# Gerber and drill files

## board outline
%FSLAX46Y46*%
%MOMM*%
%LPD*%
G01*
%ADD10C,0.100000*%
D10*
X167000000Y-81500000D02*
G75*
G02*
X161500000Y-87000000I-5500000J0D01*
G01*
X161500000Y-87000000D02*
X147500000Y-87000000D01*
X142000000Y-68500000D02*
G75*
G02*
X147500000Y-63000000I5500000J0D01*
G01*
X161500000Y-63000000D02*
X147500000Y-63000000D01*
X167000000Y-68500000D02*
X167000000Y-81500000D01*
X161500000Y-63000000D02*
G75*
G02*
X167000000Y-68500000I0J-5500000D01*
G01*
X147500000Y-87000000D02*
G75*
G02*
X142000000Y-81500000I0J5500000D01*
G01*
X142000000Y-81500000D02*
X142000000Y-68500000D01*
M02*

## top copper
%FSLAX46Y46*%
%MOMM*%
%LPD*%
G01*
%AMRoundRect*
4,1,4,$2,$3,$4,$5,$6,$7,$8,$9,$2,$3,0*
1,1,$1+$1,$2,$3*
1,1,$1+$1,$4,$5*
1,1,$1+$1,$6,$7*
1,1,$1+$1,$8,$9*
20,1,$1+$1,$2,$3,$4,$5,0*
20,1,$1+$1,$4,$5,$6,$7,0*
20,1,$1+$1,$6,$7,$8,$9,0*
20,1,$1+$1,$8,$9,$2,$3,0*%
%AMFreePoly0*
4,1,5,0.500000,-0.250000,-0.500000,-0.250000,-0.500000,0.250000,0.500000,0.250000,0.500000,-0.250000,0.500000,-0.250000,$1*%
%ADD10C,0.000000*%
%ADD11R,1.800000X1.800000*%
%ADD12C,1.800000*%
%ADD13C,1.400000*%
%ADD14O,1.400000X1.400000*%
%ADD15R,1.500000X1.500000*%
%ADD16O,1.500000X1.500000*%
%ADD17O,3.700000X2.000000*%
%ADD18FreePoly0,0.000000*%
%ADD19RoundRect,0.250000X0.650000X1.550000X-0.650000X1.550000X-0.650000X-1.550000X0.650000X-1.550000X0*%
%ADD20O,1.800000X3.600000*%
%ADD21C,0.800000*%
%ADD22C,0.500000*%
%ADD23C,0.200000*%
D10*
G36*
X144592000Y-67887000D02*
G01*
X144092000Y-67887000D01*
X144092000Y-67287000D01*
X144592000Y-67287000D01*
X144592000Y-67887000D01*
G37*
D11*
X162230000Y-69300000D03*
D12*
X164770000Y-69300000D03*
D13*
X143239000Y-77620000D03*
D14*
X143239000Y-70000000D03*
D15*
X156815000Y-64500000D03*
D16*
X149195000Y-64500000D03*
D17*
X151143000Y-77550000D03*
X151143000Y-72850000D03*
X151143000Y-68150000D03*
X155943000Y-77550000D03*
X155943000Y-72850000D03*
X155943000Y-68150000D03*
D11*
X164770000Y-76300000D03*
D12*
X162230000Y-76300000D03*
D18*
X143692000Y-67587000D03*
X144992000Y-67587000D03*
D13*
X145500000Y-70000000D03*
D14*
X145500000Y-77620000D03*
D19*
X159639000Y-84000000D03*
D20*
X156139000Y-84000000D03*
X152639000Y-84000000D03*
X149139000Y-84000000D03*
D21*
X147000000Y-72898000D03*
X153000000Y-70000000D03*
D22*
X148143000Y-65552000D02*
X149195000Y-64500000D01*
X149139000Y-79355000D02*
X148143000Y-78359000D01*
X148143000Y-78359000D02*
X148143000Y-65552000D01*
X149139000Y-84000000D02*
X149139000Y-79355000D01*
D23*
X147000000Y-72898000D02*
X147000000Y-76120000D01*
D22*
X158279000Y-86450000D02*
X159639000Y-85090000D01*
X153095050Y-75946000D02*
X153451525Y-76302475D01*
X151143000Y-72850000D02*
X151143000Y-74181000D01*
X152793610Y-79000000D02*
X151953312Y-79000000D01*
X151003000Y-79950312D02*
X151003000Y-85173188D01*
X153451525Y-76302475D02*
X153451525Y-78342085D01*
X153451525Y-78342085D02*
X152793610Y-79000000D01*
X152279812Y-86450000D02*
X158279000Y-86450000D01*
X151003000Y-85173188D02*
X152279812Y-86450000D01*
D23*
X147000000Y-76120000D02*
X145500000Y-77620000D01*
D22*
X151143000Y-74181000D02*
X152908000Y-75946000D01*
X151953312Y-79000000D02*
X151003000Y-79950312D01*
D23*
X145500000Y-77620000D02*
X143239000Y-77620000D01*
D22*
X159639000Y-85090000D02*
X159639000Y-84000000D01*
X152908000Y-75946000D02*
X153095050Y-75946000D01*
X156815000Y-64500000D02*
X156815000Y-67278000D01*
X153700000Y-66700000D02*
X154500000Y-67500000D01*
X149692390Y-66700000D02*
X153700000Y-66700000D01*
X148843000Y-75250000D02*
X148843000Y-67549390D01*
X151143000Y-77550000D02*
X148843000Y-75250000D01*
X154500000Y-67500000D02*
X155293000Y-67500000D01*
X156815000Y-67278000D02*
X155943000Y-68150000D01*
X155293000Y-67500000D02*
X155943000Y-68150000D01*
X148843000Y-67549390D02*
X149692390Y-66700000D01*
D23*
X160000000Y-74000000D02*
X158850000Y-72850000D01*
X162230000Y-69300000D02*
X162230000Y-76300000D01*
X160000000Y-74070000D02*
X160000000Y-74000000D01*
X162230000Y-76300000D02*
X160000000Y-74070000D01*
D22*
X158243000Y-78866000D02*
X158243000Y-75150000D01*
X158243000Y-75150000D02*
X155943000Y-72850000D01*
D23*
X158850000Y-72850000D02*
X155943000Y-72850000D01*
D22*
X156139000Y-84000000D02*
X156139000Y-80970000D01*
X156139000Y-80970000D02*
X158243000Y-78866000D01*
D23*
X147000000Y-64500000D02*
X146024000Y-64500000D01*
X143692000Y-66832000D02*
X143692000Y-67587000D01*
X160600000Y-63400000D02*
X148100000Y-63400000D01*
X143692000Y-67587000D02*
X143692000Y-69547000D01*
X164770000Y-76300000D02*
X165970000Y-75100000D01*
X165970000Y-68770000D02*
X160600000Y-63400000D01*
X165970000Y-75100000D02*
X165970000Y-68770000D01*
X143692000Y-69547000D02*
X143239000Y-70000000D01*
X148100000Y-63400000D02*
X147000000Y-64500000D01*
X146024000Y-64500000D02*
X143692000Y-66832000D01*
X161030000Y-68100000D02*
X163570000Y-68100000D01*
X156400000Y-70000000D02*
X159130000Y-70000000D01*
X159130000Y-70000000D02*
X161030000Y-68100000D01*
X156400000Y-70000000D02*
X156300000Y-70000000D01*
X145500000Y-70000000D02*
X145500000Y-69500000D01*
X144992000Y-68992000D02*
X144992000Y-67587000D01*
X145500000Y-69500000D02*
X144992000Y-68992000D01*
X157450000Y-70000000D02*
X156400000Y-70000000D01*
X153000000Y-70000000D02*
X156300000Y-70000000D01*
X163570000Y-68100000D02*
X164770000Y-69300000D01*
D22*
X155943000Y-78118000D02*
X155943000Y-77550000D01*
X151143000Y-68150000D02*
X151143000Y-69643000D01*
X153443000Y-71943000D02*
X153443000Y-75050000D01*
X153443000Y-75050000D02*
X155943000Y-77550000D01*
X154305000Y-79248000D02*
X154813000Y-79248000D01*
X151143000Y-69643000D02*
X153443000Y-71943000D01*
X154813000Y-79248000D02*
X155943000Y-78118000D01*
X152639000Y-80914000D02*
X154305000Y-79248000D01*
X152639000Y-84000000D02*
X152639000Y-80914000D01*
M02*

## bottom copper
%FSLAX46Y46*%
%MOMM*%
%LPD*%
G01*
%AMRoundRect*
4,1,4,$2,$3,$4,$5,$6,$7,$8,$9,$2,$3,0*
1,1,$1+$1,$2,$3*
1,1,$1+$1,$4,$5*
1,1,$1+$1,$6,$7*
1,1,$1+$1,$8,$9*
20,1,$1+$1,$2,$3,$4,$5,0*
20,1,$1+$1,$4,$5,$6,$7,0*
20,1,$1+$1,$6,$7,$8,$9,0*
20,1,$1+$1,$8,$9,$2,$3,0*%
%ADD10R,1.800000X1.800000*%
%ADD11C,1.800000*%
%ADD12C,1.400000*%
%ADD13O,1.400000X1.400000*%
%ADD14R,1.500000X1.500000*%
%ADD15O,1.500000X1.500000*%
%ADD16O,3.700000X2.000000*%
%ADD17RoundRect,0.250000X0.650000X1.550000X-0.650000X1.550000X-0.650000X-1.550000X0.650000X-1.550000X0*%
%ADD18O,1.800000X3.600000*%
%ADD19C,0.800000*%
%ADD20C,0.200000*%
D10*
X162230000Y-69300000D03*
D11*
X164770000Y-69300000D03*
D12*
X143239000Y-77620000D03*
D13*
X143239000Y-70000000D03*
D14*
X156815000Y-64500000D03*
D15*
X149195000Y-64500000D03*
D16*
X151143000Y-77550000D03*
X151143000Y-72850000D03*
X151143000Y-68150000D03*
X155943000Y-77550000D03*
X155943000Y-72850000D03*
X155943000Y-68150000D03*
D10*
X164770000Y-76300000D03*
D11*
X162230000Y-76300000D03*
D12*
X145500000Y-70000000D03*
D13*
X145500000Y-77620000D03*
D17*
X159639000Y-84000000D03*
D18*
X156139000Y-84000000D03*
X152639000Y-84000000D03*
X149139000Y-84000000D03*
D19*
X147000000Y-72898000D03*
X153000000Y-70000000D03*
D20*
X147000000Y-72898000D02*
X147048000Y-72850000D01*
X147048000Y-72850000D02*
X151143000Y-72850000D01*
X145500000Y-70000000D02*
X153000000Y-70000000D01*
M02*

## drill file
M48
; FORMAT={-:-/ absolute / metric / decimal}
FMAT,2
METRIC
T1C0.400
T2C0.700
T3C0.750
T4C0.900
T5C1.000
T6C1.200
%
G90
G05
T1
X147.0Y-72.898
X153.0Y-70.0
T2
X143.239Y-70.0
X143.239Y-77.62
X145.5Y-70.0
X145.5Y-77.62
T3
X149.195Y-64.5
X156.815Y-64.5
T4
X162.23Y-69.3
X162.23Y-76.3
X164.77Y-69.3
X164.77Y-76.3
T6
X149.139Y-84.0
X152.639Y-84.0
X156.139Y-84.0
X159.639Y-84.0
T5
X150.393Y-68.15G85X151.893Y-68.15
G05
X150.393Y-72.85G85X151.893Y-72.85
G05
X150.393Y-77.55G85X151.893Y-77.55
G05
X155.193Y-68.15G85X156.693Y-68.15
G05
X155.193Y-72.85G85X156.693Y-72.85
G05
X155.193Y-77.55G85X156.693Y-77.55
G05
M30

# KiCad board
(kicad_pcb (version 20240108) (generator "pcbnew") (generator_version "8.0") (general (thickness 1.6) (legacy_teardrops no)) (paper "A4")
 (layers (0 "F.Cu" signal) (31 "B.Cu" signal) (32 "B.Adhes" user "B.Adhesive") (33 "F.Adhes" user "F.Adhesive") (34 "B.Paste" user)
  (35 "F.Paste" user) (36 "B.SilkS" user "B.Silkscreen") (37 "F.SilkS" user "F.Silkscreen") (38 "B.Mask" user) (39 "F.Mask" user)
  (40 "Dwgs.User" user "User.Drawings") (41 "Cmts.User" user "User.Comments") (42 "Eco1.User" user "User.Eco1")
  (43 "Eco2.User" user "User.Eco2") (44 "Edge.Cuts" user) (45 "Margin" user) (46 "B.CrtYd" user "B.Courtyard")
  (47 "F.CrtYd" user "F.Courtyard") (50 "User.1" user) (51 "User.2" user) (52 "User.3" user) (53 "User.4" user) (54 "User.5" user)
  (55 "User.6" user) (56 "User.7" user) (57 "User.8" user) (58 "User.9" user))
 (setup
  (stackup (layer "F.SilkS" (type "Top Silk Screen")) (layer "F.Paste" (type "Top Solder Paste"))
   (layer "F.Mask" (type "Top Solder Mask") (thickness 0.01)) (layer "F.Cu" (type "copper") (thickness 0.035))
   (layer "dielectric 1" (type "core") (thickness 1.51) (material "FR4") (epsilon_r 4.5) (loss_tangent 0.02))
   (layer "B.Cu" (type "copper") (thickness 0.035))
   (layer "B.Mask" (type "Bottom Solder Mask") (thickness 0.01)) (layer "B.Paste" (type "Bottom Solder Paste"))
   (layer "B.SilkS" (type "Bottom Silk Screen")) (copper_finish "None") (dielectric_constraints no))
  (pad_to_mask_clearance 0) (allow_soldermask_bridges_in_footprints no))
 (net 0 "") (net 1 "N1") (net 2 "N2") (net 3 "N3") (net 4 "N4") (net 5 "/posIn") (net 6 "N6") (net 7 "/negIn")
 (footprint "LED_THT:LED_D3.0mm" (layer "F.Cu") (at 162.23 69.3)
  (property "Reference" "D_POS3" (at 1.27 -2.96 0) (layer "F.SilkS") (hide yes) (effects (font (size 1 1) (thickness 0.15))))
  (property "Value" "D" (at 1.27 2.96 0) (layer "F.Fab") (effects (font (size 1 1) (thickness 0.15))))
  (pad "1" thru_hole rect (at 0 0) (size 1.8 1.8) (drill 0.9) (layers "*.Cu" "*.Mask") (remove_unused_layers no) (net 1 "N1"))
  (pad "2" thru_hole circle (at 2.54 0) (size 1.8 1.8) (drill 0.9) (layers "*.Cu" "*.Mask") (remove_unused_layers no) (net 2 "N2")))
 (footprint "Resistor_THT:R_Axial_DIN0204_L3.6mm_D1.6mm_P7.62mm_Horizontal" (layer "F.Cu") (at 143.239 77.62 90)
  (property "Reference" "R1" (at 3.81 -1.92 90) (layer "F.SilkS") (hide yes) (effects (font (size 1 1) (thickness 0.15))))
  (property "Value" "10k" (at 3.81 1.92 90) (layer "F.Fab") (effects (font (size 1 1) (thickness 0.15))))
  (pad "1" thru_hole circle (at 0 0 90) (size 1.4 1.4) (drill 0.7) (layers "*.Cu" "*.Mask") (remove_unused_layers no) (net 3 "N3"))
  (pad "2" thru_hole oval (at 7.62 0 90) (size 1.4 1.4) (drill 0.7) (layers "*.Cu" "*.Mask") (remove_unused_layers no) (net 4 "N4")))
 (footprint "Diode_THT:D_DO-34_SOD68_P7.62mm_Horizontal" (layer "F.Cu") (at 156.815 64.5 180)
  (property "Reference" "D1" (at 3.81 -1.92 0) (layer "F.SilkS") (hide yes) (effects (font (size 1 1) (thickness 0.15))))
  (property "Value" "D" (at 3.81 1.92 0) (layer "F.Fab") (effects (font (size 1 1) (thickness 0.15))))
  (pad "1" thru_hole rect (at 0 0 180) (size 1.5 1.5) (drill 0.75) (layers "*.Cu" "*.Mask") (remove_unused_layers no) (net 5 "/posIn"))
  (pad "2" thru_hole oval (at 7.62 0 180) (size 1.5 1.5) (drill 0.75) (layers "*.Cu" "*.Mask") (remove_unused_layers no) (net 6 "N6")))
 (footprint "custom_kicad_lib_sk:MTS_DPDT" (layer "F.Cu") (at 154.143 68.85 90)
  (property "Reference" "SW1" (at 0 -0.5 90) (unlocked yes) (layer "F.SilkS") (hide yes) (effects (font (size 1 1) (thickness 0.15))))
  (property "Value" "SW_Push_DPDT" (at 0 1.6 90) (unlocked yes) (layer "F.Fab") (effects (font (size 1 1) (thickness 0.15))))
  (pad "1" thru_hole oval (at -8.7 -3 90) (size 2 3.7) (drill oval 1 2.5) (layers "*.Cu" "*.Mask") (remove_unused_layers no)
   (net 5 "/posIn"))
  (pad "2" thru_hole oval (at -4 -3 90) (size 2 3.7) (drill oval 1 2.5) (layers "*.Cu" "*.Mask") (remove_unused_layers no) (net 3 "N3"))
  (pad "3" thru_hole oval (at 0.7 -3 90) (size 2 3.7) (drill oval 1 2.5) (layers "*.Cu" "*.Mask") (remove_unused_layers no) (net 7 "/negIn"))
  (pad "4" thru_hole oval (at -8.7 1.8 90) (size 2 3.7) (drill oval 1 2.5) (layers "*.Cu" "*.Mask") (remove_unused_layers no)
   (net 7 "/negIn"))
  (pad "5" thru_hole oval (at -4 1.8 90) (size 2 3.7) (drill oval 1 2.5) (layers "*.Cu" "*.Mask") (remove_unused_layers no) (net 1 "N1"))
  (pad "6" thru_hole oval (at 0.7 1.8 90) (size 2 3.7) (drill oval 1 2.5) (layers "*.Cu" "*.Mask") (remove_unused_layers no)
   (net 5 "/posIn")))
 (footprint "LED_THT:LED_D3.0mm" (layer "F.Cu") (at 164.77 76.3 180)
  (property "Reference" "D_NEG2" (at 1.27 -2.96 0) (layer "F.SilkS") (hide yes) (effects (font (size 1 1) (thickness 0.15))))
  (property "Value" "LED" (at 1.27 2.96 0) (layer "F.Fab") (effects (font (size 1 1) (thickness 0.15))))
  (pad "1" thru_hole rect (at 0 0 180) (size 1.8 1.8) (drill 0.9) (layers "*.Cu" "*.Mask") (remove_unused_layers no) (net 4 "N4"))
  (pad "2" thru_hole circle (at 2.54 0 180) (size 1.8 1.8) (drill 0.9) (layers "*.Cu" "*.Mask") (remove_unused_layers no) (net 1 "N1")))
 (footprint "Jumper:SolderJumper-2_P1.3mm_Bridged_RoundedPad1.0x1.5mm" (layer "F.Cu") (at 144.342 67.587)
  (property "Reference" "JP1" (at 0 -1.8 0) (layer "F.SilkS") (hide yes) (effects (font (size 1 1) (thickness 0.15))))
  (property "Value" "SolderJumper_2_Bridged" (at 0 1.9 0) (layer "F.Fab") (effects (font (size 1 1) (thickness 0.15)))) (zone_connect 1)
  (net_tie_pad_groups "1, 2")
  (fp_poly (pts (xy 0.25 -0.3) (xy -0.25 -0.3) (xy -0.25 0.3) (xy 0.25 0.3)) (stroke (width 0) (type solid)) (fill solid) (layer "F.Cu"))
  (pad "1" smd custom (at -0.65 0) (size 1 0.5) (layers "F.Cu" "F.Mask") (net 4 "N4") (zone_connect 2) (thermal_bridge_angle 45)
   (options (clearance outline) (anchor rect)) (primitives))
  (pad "2" smd custom (at 0.65 0) (size 1 0.5) (layers "F.Cu" "F.Mask") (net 2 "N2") (zone_connect 2) (thermal_bridge_angle 45)
   (options (clearance outline) (anchor rect)) (primitives)))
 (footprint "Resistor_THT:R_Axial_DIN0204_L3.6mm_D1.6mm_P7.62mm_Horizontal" (layer "F.Cu") (at 145.5 70 -90)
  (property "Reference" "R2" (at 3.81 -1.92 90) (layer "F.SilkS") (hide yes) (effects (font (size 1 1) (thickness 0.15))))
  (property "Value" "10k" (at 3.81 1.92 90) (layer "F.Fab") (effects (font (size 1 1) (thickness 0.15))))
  (pad "1" thru_hole circle (at 0 0 270) (size 1.4 1.4) (drill 0.7) (layers "*.Cu" "*.Mask") (remove_unused_layers no) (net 2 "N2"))
  (pad "2" thru_hole oval (at 7.62 0 270) (size 1.4 1.4) (drill 0.7) (layers "*.Cu" "*.Mask") (remove_unused_layers no) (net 3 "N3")))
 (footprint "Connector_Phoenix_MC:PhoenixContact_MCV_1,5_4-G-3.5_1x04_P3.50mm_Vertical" (layer "B.Cu") (at 159.639 84 180)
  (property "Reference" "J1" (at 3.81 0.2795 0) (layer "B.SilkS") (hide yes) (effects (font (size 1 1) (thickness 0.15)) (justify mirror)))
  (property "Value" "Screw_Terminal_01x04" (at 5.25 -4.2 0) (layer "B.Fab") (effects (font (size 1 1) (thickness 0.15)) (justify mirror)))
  (pad "1" thru_hole roundrect (at 0 0 180) (size 1.8 3.6) (drill 1.2) (layers "*.Cu" "*.Mask") (remove_unused_layers no)
   (roundrect_rratio 0.138889) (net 3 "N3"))
  (pad "2" thru_hole oval (at 3.5 0 180) (size 1.8 3.6) (drill 1.2) (layers "*.Cu" "*.Mask") (remove_unused_layers no) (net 1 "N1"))
  (pad "3" thru_hole oval (at 7 0 180) (size 1.8 3.6) (drill 1.2) (layers "*.Cu" "*.Mask") (remove_unused_layers no) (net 7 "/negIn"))
  (pad "4" thru_hole oval (at 10.5 0 180) (size 1.8 3.6) (drill 1.2) (layers "*.Cu" "*.Mask") (remove_unused_layers no) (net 6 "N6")))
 (gr_arc (start 167 81.5) (mid 165.389087 85.389087) (end 161.5 87) (stroke (width 0.1) (type default)) (layer "Edge.Cuts"))
 (gr_line (start 161.5 87) (end 147.5 87) (stroke (width 0.1) (type default)) (layer "Edge.Cuts"))
 (gr_arc (start 142 68.5) (mid 143.610913 64.610913) (end 147.5 63) (stroke (width 0.1) (type default)) (layer "Edge.Cuts"))
 (gr_line (start 161.5 63) (end 147.5 63) (stroke (width 0.1) (type default)) (layer "Edge.Cuts"))
 (gr_line (start 167 68.5) (end 167 81.5) (stroke (width 0.1) (type default)) (layer "Edge.Cuts"))
 (gr_arc (start 161.5 63) (mid 165.389087 64.610913) (end 167 68.5) (stroke (width 0.1) (type default)) (layer "Edge.Cuts"))
 (gr_arc (start 147.5 87) (mid 143.610913 85.389087) (end 142 81.5) (stroke (width 0.1) (type default)) (layer "Edge.Cuts"))
 (gr_line (start 142 81.5) (end 142 68.5) (stroke (width 0.1) (type default)) (layer "Edge.Cuts"))
 (segment (start 148.143 65.552) (end 149.195 64.5) (width 0.5) (layer "F.Cu") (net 6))
 (segment (start 149.139 79.355) (end 148.143 78.359) (width 0.5) (layer "F.Cu") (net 6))
 (segment (start 148.143 78.359) (end 148.143 65.552) (width 0.5) (layer "F.Cu") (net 6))
 (segment (start 149.139 84) (end 149.139 79.355) (width 0.5) (layer "F.Cu") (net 6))
 (segment (start 147 72.898) (end 147 76.12) (width 0.2) (layer "F.Cu") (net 3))
 (segment (start 158.279 86.45) (end 159.639 85.09) (width 0.5) (layer "F.Cu") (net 3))
 (segment (start 153.09505 75.946) (end 153.451525 76.302475) (width 0.5) (layer "F.Cu") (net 3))
 (segment (start 151.143 72.85) (end 151.143 74.181) (width 0.5) (layer "F.Cu") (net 3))
 (segment (start 152.79361 79) (end 151.953312 79) (width 0.5) (layer "F.Cu") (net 3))
 (segment (start 151.003 79.950312) (end 151.003 85.173188) (width 0.5) (layer "F.Cu") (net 3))
 (segment (start 153.451525 76.302475) (end 153.451525 78.342085) (width 0.5) (layer "F.Cu") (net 3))
 (segment (start 153.451525 78.342085) (end 152.79361 79) (width 0.5) (layer "F.Cu") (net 3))
 (segment (start 152.279812 86.45) (end 158.279 86.45) (width 0.5) (layer "F.Cu") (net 3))
 (segment (start 151.003 85.173188) (end 152.279812 86.45) (width 0.5) (layer "F.Cu") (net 3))
 (segment (start 147 76.12) (end 145.5 77.62) (width 0.2) (layer "F.Cu") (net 3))
 (segment (start 151.143 74.181) (end 152.908 75.946) (width 0.5) (layer "F.Cu") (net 3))
 (segment (start 151.953312 79) (end 151.003 79.950312) (width 0.5) (layer "F.Cu") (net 3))
 (segment (start 145.5 77.62) (end 143.239 77.62) (width 0.2) (layer "F.Cu") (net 3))
 (segment (start 159.639 85.09) (end 159.639 84) (width 0.5) (layer "F.Cu") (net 3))
 (segment (start 152.908 75.946) (end 153.09505 75.946) (width 0.5) (layer "F.Cu") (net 3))
 (via (at 147 72.898) (size 0.8) (drill 0.4) (layers "F.Cu" "B.Cu") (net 3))
 (segment (start 147 72.898) (end 147.048 72.85) (width 0.2) (layer "B.Cu") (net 3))
 (segment (start 147.048 72.85) (end 151.143 72.85) (width 0.2) (layer "B.Cu") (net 3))
 (segment (start 156.815 64.5) (end 156.815 67.278) (width 0.5) (layer "F.Cu") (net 5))
 (segment (start 153.7 66.7) (end 154.5 67.5) (width 0.5) (layer "F.Cu") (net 5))
 (segment (start 149.69239 66.7) (end 153.7 66.7) (width 0.5) (layer "F.Cu") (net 5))
 (segment (start 148.843 75.25) (end 148.843 67.54939) (width 0.5) (layer "F.Cu") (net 5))
 (segment (start 151.143 77.55) (end 148.843 75.25) (width 0.5) (layer "F.Cu") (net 5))
 (segment (start 154.5 67.5) (end 155.293 67.5) (width 0.5) (layer "F.Cu") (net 5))
 (segment (start 156.815 67.278) (end 155.943 68.15) (width 0.5) (layer "F.Cu") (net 5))
 (segment (start 155.293 67.5) (end 155.943 68.15) (width 0.5) (layer "F.Cu") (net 5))
 (segment (start 148.843 67.54939) (end 149.69239 66.7) (width 0.5) (layer "F.Cu") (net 5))
 (segment (start 160 74) (end 158.85 72.85) (width 0.2) (layer "F.Cu") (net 1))
 (segment (start 162.23 69.3) (end 162.23 76.3) (width 0.2) (layer "F.Cu") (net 1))
 (segment (start 160 74.07) (end 160 74) (width 0.2) (layer "F.Cu") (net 1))
 (segment (start 162.23 76.3) (end 160 74.07) (width 0.2) (layer "F.Cu") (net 1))
 (segment (start 158.243 78.866) (end 158.243 75.15) (width 0.5) (layer "F.Cu") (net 1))
 (segment (start 158.243 75.15) (end 155.943 72.85) (width 0.5) (layer "F.Cu") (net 1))
 (segment (start 158.85 72.85) (end 155.943 72.85) (width 0.2) (layer "F.Cu") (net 1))
 (segment (start 156.139 84) (end 156.139 80.97) (width 0.5) (layer "F.Cu") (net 1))
 (segment (start 156.139 80.97) (end 158.243 78.866) (width 0.5) (layer "F.Cu") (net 1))
 (segment (start 147 64.5) (end 146.024 64.5) (width 0.2) (layer "F.Cu") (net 4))
 (segment (start 143.692 66.832) (end 143.692 67.587) (width 0.2) (layer "F.Cu") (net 4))
 (segment (start 160.6 63.4) (end 148.1 63.4) (width 0.2) (layer "F.Cu") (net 4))
 (segment (start 143.692 67.587) (end 143.692 69.547) (width 0.2) (layer "F.Cu") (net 4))
 (segment (start 164.77 76.3) (end 165.97 75.1) (width 0.2) (layer "F.Cu") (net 4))
 (segment (start 165.97 68.77) (end 160.6 63.4) (width 0.2) (layer "F.Cu") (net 4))
 (segment (start 165.97 75.1) (end 165.97 68.77) (width 0.2) (layer "F.Cu") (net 4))
 (segment (start 143.692 69.547) (end 143.239 70) (width 0.2) (layer "F.Cu") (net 4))
 (segment (start 148.1 63.4) (end 147 64.5) (width 0.2) (layer "F.Cu") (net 4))
 (segment (start 146.024 64.5) (end 143.692 66.832) (width 0.2) (layer "F.Cu") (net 4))
 (segment (start 161.03 68.1) (end 163.57 68.1) (width 0.2) (layer "F.Cu") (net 2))
 (segment (start 156.4 70) (end 159.13 70) (width 0.2) (layer "F.Cu") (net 2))
 (segment (start 159.13 70) (end 161.03 68.1) (width 0.2) (layer "F.Cu") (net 2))
 (segment (start 156.4 70) (end 156.3 70) (width 0.2) (layer "F.Cu") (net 2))
 (segment (start 145.5 70) (end 145.5 69.5) (width 0.2) (layer "F.Cu") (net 2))
 (segment (start 144.992 68.992) (end 144.992 67.587) (width 0.2) (layer "F.Cu") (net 2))
 (segment (start 145.5 69.5) (end 144.992 68.992) (width 0.2) (layer "F.Cu") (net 2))
 (segment (start 157.45 70) (end 156.4 70) (width 0.2) (layer "F.Cu") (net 2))
 (segment (start 153 70) (end 156.3 70) (width 0.2) (layer "F.Cu") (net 2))
 (segment (start 163.57 68.1) (end 164.77 69.3) (width 0.2) (layer "F.Cu") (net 2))
 (via (at 153 70) (size 0.8) (drill 0.4) (layers "F.Cu" "B.Cu") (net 2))
 (segment (start 145.5 70) (end 153 70) (width 0.2) (layer "B.Cu") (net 2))
 (segment (start 155.943 78.118) (end 155.943 77.55) (width 0.5) (layer "F.Cu") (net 7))
 (segment (start 151.143 68.15) (end 151.143 69.643) (width 0.5) (layer "F.Cu") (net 7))
 (segment (start 153.443 71.943) (end 153.443 75.05) (width 0.5) (layer "F.Cu") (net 7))
 (segment (start 153.443 75.05) (end 155.943 77.55) (width 0.5) (layer "F.Cu") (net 7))
 (segment (start 154.305 79.248) (end 154.813 79.248) (width 0.5) (layer "F.Cu") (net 7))
 (segment (start 151.143 69.643) (end 153.443 71.943) (width 0.5) (layer "F.Cu") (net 7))
 (segment (start 154.813 79.248) (end 155.943 78.118) (width 0.5) (layer "F.Cu") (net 7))
 (segment (start 152.639 80.914) (end 154.305 79.248) (width 0.5) (layer "F.Cu") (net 7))
 (segment (start 152.639 84) (end 152.639 80.914) (width 0.5) (layer "F.Cu") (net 7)))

